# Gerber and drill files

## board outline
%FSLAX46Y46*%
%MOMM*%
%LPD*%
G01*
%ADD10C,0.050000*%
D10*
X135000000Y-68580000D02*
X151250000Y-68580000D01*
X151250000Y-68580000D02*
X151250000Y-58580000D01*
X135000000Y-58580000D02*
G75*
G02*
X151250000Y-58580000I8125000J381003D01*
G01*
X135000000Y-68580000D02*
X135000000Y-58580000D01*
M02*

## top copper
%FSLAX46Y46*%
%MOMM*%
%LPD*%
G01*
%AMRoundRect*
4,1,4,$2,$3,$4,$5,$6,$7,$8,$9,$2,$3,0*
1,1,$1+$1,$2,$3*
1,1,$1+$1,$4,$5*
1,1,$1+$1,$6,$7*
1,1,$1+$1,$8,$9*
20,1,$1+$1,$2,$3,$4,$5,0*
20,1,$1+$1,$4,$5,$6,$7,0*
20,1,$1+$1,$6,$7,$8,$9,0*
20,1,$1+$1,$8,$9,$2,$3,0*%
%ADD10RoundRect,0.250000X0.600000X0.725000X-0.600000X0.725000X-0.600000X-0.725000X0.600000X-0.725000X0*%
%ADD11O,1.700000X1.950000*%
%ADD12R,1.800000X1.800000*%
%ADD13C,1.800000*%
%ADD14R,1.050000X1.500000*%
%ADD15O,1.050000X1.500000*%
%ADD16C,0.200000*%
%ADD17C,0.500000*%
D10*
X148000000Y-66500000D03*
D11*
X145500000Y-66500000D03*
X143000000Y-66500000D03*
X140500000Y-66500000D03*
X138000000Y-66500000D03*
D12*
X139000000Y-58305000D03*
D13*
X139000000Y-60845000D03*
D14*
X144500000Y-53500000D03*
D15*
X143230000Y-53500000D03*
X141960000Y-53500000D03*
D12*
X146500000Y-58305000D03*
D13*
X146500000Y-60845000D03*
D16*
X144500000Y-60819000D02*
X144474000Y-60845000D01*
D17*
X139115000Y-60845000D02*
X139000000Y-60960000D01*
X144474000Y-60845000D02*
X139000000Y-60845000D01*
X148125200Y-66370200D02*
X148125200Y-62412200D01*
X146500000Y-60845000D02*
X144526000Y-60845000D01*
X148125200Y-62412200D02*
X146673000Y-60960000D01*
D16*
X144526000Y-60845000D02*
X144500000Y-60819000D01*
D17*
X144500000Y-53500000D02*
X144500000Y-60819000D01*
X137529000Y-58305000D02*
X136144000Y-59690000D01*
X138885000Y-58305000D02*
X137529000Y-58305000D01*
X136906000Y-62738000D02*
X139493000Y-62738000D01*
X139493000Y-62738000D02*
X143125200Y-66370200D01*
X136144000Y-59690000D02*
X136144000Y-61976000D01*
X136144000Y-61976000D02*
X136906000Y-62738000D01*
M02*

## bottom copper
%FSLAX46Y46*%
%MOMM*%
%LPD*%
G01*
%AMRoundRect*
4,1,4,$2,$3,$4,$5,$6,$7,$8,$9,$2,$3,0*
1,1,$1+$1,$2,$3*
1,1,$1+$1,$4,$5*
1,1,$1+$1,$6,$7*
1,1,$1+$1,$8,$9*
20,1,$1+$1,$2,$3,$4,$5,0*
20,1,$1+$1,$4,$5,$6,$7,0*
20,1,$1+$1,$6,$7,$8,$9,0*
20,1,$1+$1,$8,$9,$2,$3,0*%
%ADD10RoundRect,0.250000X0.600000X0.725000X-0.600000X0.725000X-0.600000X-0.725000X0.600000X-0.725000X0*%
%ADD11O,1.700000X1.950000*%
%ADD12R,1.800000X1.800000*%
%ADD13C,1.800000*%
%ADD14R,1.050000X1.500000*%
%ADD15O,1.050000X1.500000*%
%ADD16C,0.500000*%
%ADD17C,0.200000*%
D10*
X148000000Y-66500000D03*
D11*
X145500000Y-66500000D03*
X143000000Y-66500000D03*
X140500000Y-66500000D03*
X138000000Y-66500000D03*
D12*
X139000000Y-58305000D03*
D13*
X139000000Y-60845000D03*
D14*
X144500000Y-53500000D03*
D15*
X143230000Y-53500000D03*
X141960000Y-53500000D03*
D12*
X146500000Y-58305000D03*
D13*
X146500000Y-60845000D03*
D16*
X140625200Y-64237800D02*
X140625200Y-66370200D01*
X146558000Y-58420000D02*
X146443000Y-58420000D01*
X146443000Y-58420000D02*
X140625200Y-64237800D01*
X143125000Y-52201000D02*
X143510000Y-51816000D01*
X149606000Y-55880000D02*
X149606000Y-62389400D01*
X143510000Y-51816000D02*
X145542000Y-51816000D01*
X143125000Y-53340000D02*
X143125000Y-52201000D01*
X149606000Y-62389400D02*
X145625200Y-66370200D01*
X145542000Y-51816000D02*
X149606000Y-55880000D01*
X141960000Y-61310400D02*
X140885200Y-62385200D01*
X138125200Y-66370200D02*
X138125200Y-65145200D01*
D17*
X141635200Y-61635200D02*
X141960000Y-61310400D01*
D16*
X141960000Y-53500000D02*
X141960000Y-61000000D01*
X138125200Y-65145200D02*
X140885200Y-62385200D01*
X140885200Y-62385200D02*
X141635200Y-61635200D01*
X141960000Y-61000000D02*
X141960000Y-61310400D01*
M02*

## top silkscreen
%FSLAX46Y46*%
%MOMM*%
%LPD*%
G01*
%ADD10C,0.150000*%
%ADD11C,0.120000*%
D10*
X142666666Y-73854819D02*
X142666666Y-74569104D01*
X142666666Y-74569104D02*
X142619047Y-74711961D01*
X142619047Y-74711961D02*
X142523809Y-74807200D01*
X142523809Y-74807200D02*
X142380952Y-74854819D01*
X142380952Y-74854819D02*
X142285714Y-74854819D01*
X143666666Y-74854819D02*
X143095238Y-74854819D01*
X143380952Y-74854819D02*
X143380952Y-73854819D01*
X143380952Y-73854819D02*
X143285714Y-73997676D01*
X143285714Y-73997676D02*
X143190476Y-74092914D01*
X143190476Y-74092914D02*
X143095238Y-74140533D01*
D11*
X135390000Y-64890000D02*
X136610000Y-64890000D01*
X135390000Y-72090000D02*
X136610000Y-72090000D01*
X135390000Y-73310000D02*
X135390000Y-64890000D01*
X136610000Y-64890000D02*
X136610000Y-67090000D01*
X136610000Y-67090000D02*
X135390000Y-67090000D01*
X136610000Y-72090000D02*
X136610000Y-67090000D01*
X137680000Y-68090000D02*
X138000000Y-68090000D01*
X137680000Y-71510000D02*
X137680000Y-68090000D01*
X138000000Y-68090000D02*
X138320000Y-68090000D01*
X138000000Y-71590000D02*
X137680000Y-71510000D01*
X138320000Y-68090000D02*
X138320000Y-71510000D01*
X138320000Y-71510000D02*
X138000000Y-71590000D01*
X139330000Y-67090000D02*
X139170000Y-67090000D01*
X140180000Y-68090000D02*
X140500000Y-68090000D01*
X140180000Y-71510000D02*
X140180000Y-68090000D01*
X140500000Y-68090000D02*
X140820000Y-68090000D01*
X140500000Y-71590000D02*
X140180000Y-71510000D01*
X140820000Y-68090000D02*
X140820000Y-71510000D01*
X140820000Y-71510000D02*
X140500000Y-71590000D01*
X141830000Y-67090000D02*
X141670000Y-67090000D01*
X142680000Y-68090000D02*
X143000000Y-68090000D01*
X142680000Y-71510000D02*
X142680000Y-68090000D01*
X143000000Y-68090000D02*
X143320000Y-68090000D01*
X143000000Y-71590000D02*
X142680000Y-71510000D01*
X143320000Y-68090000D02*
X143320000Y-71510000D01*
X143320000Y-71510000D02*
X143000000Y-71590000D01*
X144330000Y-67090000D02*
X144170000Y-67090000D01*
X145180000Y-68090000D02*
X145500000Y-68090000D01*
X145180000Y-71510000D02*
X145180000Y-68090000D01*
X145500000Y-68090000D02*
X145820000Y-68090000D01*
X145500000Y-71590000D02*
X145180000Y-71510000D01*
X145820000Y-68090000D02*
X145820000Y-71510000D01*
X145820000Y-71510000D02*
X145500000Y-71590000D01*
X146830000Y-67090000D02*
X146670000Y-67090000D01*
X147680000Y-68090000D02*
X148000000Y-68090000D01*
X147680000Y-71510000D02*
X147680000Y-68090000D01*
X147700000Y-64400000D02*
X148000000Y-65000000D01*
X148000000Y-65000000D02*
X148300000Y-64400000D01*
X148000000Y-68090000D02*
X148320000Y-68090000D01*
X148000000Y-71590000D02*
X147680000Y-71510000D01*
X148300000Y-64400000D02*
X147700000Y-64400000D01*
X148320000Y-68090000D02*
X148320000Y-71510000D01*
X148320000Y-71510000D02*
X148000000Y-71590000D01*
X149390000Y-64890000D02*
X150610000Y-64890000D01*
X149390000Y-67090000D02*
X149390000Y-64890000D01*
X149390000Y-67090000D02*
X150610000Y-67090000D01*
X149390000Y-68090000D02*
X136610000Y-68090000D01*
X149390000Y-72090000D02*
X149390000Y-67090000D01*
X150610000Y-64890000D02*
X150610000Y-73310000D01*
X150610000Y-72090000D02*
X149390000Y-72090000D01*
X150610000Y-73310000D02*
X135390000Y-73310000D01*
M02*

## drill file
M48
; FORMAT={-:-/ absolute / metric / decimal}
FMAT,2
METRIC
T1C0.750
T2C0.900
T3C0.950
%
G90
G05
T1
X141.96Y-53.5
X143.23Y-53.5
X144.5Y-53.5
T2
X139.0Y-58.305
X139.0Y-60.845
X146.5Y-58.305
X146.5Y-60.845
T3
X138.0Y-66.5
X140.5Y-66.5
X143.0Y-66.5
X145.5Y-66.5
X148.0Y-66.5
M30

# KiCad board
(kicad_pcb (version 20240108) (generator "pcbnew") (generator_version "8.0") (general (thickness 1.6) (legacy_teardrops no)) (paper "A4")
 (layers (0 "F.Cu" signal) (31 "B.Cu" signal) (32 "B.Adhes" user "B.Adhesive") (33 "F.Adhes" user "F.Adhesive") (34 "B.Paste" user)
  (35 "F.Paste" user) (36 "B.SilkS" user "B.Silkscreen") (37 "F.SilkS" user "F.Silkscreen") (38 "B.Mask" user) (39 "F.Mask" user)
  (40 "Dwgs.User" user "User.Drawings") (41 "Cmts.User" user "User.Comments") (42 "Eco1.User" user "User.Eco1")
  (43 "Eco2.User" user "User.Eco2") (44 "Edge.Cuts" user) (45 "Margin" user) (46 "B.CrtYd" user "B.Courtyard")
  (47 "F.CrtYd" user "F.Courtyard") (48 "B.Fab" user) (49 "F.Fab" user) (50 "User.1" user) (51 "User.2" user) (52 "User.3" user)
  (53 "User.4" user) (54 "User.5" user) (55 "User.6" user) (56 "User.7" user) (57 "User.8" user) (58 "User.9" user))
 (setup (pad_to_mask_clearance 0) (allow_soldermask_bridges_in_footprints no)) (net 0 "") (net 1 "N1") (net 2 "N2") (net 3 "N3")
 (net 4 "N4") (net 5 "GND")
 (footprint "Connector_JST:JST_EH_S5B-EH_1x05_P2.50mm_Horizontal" (layer "F.Cu") (at 148 66.5 180)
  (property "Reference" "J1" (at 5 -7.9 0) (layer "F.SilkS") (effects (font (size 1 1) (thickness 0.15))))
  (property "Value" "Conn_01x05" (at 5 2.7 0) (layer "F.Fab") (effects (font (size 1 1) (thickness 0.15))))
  (fp_line (start 12.61 1.61) (end 11.39 1.61) (stroke (width 0.12) (type solid)) (layer "F.SilkS"))
  (fp_line (start 12.61 -5.59) (end 11.39 -5.59) (stroke (width 0.12) (type solid)) (layer "F.SilkS"))
  (fp_line (start 12.61 -6.81) (end 12.61 1.61) (stroke (width 0.12) (type solid)) (layer "F.SilkS"))
  (fp_line (start 11.39 1.61) (end 11.39 -0.59) (stroke (width 0.12) (type solid)) (layer "F.SilkS"))
  (fp_line (start 11.39 -0.59) (end 12.61 -0.59) (stroke (width 0.12) (type solid)) (layer "F.SilkS"))
  (fp_line (start 11.39 -5.59) (end 11.39 -0.59) (stroke (width 0.12) (type solid)) (layer "F.SilkS"))
  (fp_line (start 10.32 -1.59) (end 10 -1.59) (stroke (width 0.12) (type solid)) (layer "F.SilkS"))
  (fp_line (start 10.32 -5.01) (end 10.32 -1.59) (stroke (width 0.12) (type solid)) (layer "F.SilkS"))
  (fp_line (start 10 -1.59) (end 9.68 -1.59) (stroke (width 0.12) (type solid)) (layer "F.SilkS"))
  (fp_line (start 10 -5.09) (end 10.32 -5.01) (stroke (width 0.12) (type solid)) (layer "F.SilkS"))
  (fp_line (start 9.68 -1.59) (end 9.68 -5.01) (stroke (width 0.12) (type solid)) (layer "F.SilkS"))
  (fp_line (start 9.68 -5.01) (end 10 -5.09) (stroke (width 0.12) (type solid)) (layer "F.SilkS"))
  (fp_line (start 8.67 -0.59) (end 8.83 -0.59) (stroke (width 0.12) (type solid)) (layer "F.SilkS"))
  (fp_line (start 7.82 -1.59) (end 7.5 -1.59) (stroke (width 0.12) (type solid)) (layer "F.SilkS"))
  (fp_line (start 7.82 -5.01) (end 7.82 -1.59) (stroke (width 0.12) (type solid)) (layer "F.SilkS"))
  (fp_line (start 7.5 -1.59) (end 7.18 -1.59) (stroke (width 0.12) (type solid)) (layer "F.SilkS"))
  (fp_line (start 7.5 -5.09) (end 7.82 -5.01) (stroke (width 0.12) (type solid)) (layer "F.SilkS"))
  (fp_line (start 7.18 -1.59) (end 7.18 -5.01) (stroke (width 0.12) (type solid)) (layer "F.SilkS"))
  (fp_line (start 7.18 -5.01) (end 7.5 -5.09) (stroke (width 0.12) (type solid)) (layer "F.SilkS"))
  (fp_line (start 6.17 -0.59) (end 6.33 -0.59) (stroke (width 0.12) (type solid)) (layer "F.SilkS"))
  (fp_line (start 5.32 -1.59) (end 5 -1.59) (stroke (width 0.12) (type solid)) (layer "F.SilkS"))
  (fp_line (start 5.32 -5.01) (end 5.32 -1.59) (stroke (width 0.12) (type solid)) (layer "F.SilkS"))
  (fp_line (start 5 -1.59) (end 4.68 -1.59) (stroke (width 0.12) (type solid)) (layer "F.SilkS"))
  (fp_line (start 5 -5.09) (end 5.32 -5.01) (stroke (width 0.12) (type solid)) (layer "F.SilkS"))
  (fp_line (start 4.68 -1.59) (end 4.68 -5.01) (stroke (width 0.12) (type solid)) (layer "F.SilkS"))
  (fp_line (start 4.68 -5.01) (end 5 -5.09) (stroke (width 0.12) (type solid)) (layer "F.SilkS"))
  (fp_line (start 3.67 -0.59) (end 3.83 -0.59) (stroke (width 0.12) (type solid)) (layer "F.SilkS"))
  (fp_line (start 2.82 -1.59) (end 2.5 -1.59) (stroke (width 0.12) (type solid)) (layer "F.SilkS"))
  (fp_line (start 2.82 -5.01) (end 2.82 -1.59) (stroke (width 0.12) (type solid)) (layer "F.SilkS"))
  (fp_line (start 2.5 -1.59) (end 2.18 -1.59) (stroke (width 0.12) (type solid)) (layer "F.SilkS"))
  (fp_line (start 2.5 -5.09) (end 2.82 -5.01) (stroke (width 0.12) (type solid)) (layer "F.SilkS"))
  (fp_line (start 2.18 -1.59) (end 2.18 -5.01) (stroke (width 0.12) (type solid)) (layer "F.SilkS"))
  (fp_line (start 2.18 -5.01) (end 2.5 -5.09) (stroke (width 0.12) (type solid)) (layer "F.SilkS"))
  (fp_line (start 1.17 -0.59) (end 1.33 -0.59) (stroke (width 0.12) (type solid)) (layer "F.SilkS"))
  (fp_line (start 0.32 -1.59) (end 0 -1.59) (stroke (width 0.12) (type solid)) (layer "F.SilkS"))
  (fp_line (start 0.32 -5.01) (end 0.32 -1.59) (stroke (width 0.12) (type solid)) (layer "F.SilkS"))
  (fp_line (start 0.3 2.1) (end 0 1.5) (stroke (width 0.12) (type solid)) (layer "F.SilkS"))
  (fp_line (start 0 1.5) (end -0.3 2.1) (stroke (width 0.12) (type solid)) (layer "F.SilkS"))
  (fp_line (start 0 -1.59) (end -0.32 -1.59) (stroke (width 0.12) (type solid)) (layer "F.SilkS"))
  (fp_line (start 0 -5.09) (end 0.32 -5.01) (stroke (width 0.12) (type solid)) (layer "F.SilkS"))
  (fp_line (start -0.3 2.1) (end 0.3 2.1) (stroke (width 0.12) (type solid)) (layer "F.SilkS"))
  (fp_line (start -0.32 -1.59) (end -0.32 -5.01) (stroke (width 0.12) (type solid)) (layer "F.SilkS"))
  (fp_line (start -0.32 -5.01) (end 0 -5.09) (stroke (width 0.12) (type solid)) (layer "F.SilkS"))
  (fp_line (start -1.39 1.61) (end -2.61 1.61) (stroke (width 0.12) (type solid)) (layer "F.SilkS"))
  (fp_line (start -1.39 -0.59) (end -1.39 1.61) (stroke (width 0.12) (type solid)) (layer "F.SilkS"))
  (fp_line (start -1.39 -0.59) (end -2.61 -0.59) (stroke (width 0.12) (type solid)) (layer "F.SilkS"))
  (fp_line (start -1.39 -1.59) (end 11.39 -1.59) (stroke (width 0.12) (type solid)) (layer "F.SilkS"))
  (fp_line (start -1.39 -5.59) (end -1.39 -0.59) (stroke (width 0.12) (type solid)) (layer "F.SilkS"))
  (fp_line (start -2.61 1.61) (end -2.61 -6.81) (stroke (width 0.12) (type solid)) (layer "F.SilkS"))
  (fp_line (start -2.61 -5.59) (end -1.39 -5.59) (stroke (width 0.12) (type solid)) (layer "F.SilkS"))
  (fp_line (start -2.61 -6.81) (end 12.61 -6.81) (stroke (width 0.12) (type solid)) (layer "F.SilkS"))
  (pad "1" thru_hole roundrect (at 0 0 180) (size 1.7 1.95) (drill 0.95) (layers "*.Cu" "*.Mask") (remove_unused_layers no)
   (roundrect_rratio 0.147059) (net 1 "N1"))
  (pad "2" thru_hole oval (at 2.5 0 180) (size 1.7 1.95) (drill 0.95) (layers "*.Cu" "*.Mask") (remove_unused_layers no) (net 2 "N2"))
  (pad "3" thru_hole oval (at 5 0 180) (size 1.7 1.95) (drill 0.95) (layers "*.Cu" "*.Mask") (remove_unused_layers no) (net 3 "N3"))
  (pad "4" thru_hole oval (at 7.5 0 180) (size 1.7 1.95) (drill 0.95) (layers "*.Cu" "*.Mask") (remove_unused_layers no) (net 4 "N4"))
  (pad "5" thru_hole oval (at 10 0 180) (size 1.7 1.95) (drill 0.95) (layers "*.Cu" "*.Mask") (remove_unused_layers no) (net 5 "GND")))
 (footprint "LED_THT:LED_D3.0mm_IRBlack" (layer "B.Cu") (at 139 58.305 -90)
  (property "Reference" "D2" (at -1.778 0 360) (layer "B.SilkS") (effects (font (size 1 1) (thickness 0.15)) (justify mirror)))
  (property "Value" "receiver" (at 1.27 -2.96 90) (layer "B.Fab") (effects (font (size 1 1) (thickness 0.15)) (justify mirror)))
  (pad "1" thru_hole rect (at 0 0 270) (size 1.8 1.8) (drill 0.9) (layers "*.Cu" "*.Mask") (remove_unused_layers no) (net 3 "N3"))
  (pad "2" thru_hole circle (at 2.54 0 270) (size 1.8 1.8) (drill 0.9) (layers "*.Cu" "*.Mask") (remove_unused_layers no) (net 1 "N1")))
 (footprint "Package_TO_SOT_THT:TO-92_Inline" (layer "B.Cu") (at 144.5 53.5 180)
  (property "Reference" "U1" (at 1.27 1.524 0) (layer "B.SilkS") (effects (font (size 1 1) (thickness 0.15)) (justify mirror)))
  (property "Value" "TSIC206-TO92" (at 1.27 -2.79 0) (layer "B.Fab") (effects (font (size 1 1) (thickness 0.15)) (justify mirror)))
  (pad "1" thru_hole rect (at 0 0 180) (size 1.05 1.5) (drill 0.75) (layers "*.Cu" "*.Mask") (remove_unused_layers no) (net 1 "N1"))
  (pad "2" thru_hole oval (at 1.27 0 180) (size 1.05 1.5) (drill 0.75) (layers "*.Cu" "*.Mask") (remove_unused_layers no) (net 2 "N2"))
  (pad "3" thru_hole oval (at 2.54 0 180) (size 1.05 1.5) (drill 0.75) (layers "*.Cu" "*.Mask") (remove_unused_layers no) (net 5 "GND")))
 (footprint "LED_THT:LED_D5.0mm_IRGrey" (layer "B.Cu") (at 146.5 58.305 -90)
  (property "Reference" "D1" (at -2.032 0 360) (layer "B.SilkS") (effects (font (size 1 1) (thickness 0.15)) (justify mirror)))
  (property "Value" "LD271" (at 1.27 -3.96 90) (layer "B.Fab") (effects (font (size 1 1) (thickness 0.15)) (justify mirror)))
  (pad "1" thru_hole rect (at 0 0 270) (size 1.8 1.8) (drill 0.9) (layers "*.Cu" "*.Mask") (remove_unused_layers no) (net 4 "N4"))
  (pad "2" thru_hole circle (at 2.54 0 270) (size 1.8 1.8) (drill 0.9) (layers "*.Cu" "*.Mask") (remove_unused_layers no) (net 1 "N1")))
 (gr_line (start 135 68.58) (end 151.25 68.58) (stroke (width 0.05) (type default)) (layer "Edge.Cuts"))
 (gr_line (start 151.25 68.58) (end 151.25 58.58) (stroke (width 0.05) (type default)) (layer "Edge.Cuts"))
 (gr_arc (start 135 58.58) (mid 143.125 50.065069) (end 151.25 58.58) (stroke (width 0.05) (type default)) (layer "Edge.Cuts"))
 (gr_line (start 135 68.58) (end 135 58.58) (stroke (width 0.05) (type default)) (layer "Edge.Cuts"))
 (segment (start 140.6252 64.2378) (end 140.6252 66.3702) (width 0.5) (layer "B.Cu") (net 4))
 (segment (start 146.558 58.42) (end 146.443 58.42) (width 0.5) (layer "B.Cu") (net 4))
 (segment (start 146.443 58.42) (end 140.6252 64.2378) (width 0.5) (layer "B.Cu") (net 4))
 (segment (start 144.5 60.819) (end 144.474 60.845) (width 0.2) (layer "F.Cu") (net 1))
 (segment (start 139.115 60.845) (end 139 60.96) (width 0.5) (layer "F.Cu") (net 1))
 (segment (start 144.474 60.845) (end 139 60.845) (width 0.5) (layer "F.Cu") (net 1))
 (segment (start 148.1252 66.3702) (end 148.1252 62.4122) (width 0.5) (layer "F.Cu") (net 1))
 (segment (start 146.5 60.845) (end 144.526 60.845) (width 0.5) (layer "F.Cu") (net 1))
 (segment (start 148.1252 62.4122) (end 146.673 60.96) (width 0.5) (layer "F.Cu") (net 1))
 (segment (start 144.526 60.845) (end 144.5 60.819) (width 0.2) (layer "F.Cu") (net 1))
 (segment (start 144.5 53.5) (end 144.5 60.819) (width 0.5) (layer "F.Cu") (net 1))
 (segment (start 137.529 58.305) (end 136.144 59.69) (width 0.5) (layer "F.Cu") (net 3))
 (segment (start 138.885 58.305) (end 137.529 58.305) (width 0.5) (layer "F.Cu") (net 3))
 (segment (start 136.906 62.738) (end 139.493 62.738) (width 0.5) (layer "F.Cu") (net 3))
 (segment (start 139.493 62.738) (end 143.1252 66.3702) (width 0.5) (layer "F.Cu") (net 3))
 (segment (start 136.144 59.69) (end 136.144 61.976) (width 0.5) (layer "F.Cu") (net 3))
 (segment (start 136.144 61.976) (end 136.906 62.738) (width 0.5) (layer "F.Cu") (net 3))
 (segment (start 143.125 52.201) (end 143.51 51.816) (width 0.5) (layer "B.Cu") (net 2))
 (segment (start 149.606 55.88) (end 149.606 62.3894) (width 0.5) (layer "B.Cu") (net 2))
 (segment (start 143.51 51.816) (end 145.542 51.816) (width 0.5) (layer "B.Cu") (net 2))
 (segment (start 143.125 53.34) (end 143.125 52.201) (width 0.5) (layer "B.Cu") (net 2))
 (segment (start 149.606 62.3894) (end 145.6252 66.3702) (width 0.5) (layer "B.Cu") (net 2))
 (segment (start 145.542 51.816) (end 149.606 55.88) (width 0.5) (layer "B.Cu") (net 2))
 (segment (start 141.96 61.3104) (end 140.8852 62.3852) (width 0.5) (layer "B.Cu") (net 5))
 (segment (start 138.1252 66.3702) (end 138.1252 65.1452) (width 0.5) (layer "B.Cu") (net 5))
 (segment (start 141.6352 61.6352) (end 141.96 61.3104) (width 0.2) (layer "B.Cu") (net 5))
 (segment (start 141.96 53.5) (end 141.96 61) (width 0.5) (layer "B.Cu") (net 5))
 (segment (start 138.1252 65.1452) (end 140.8852 62.3852) (width 0.5) (layer "B.Cu") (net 5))
 (segment (start 140.8852 62.3852) (end 141.6352 61.6352) (width 0.5) (layer "B.Cu") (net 5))
 (segment (start 141.96 61) (end 141.96 61.3104) (width 0.5) (layer "B.Cu") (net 5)))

